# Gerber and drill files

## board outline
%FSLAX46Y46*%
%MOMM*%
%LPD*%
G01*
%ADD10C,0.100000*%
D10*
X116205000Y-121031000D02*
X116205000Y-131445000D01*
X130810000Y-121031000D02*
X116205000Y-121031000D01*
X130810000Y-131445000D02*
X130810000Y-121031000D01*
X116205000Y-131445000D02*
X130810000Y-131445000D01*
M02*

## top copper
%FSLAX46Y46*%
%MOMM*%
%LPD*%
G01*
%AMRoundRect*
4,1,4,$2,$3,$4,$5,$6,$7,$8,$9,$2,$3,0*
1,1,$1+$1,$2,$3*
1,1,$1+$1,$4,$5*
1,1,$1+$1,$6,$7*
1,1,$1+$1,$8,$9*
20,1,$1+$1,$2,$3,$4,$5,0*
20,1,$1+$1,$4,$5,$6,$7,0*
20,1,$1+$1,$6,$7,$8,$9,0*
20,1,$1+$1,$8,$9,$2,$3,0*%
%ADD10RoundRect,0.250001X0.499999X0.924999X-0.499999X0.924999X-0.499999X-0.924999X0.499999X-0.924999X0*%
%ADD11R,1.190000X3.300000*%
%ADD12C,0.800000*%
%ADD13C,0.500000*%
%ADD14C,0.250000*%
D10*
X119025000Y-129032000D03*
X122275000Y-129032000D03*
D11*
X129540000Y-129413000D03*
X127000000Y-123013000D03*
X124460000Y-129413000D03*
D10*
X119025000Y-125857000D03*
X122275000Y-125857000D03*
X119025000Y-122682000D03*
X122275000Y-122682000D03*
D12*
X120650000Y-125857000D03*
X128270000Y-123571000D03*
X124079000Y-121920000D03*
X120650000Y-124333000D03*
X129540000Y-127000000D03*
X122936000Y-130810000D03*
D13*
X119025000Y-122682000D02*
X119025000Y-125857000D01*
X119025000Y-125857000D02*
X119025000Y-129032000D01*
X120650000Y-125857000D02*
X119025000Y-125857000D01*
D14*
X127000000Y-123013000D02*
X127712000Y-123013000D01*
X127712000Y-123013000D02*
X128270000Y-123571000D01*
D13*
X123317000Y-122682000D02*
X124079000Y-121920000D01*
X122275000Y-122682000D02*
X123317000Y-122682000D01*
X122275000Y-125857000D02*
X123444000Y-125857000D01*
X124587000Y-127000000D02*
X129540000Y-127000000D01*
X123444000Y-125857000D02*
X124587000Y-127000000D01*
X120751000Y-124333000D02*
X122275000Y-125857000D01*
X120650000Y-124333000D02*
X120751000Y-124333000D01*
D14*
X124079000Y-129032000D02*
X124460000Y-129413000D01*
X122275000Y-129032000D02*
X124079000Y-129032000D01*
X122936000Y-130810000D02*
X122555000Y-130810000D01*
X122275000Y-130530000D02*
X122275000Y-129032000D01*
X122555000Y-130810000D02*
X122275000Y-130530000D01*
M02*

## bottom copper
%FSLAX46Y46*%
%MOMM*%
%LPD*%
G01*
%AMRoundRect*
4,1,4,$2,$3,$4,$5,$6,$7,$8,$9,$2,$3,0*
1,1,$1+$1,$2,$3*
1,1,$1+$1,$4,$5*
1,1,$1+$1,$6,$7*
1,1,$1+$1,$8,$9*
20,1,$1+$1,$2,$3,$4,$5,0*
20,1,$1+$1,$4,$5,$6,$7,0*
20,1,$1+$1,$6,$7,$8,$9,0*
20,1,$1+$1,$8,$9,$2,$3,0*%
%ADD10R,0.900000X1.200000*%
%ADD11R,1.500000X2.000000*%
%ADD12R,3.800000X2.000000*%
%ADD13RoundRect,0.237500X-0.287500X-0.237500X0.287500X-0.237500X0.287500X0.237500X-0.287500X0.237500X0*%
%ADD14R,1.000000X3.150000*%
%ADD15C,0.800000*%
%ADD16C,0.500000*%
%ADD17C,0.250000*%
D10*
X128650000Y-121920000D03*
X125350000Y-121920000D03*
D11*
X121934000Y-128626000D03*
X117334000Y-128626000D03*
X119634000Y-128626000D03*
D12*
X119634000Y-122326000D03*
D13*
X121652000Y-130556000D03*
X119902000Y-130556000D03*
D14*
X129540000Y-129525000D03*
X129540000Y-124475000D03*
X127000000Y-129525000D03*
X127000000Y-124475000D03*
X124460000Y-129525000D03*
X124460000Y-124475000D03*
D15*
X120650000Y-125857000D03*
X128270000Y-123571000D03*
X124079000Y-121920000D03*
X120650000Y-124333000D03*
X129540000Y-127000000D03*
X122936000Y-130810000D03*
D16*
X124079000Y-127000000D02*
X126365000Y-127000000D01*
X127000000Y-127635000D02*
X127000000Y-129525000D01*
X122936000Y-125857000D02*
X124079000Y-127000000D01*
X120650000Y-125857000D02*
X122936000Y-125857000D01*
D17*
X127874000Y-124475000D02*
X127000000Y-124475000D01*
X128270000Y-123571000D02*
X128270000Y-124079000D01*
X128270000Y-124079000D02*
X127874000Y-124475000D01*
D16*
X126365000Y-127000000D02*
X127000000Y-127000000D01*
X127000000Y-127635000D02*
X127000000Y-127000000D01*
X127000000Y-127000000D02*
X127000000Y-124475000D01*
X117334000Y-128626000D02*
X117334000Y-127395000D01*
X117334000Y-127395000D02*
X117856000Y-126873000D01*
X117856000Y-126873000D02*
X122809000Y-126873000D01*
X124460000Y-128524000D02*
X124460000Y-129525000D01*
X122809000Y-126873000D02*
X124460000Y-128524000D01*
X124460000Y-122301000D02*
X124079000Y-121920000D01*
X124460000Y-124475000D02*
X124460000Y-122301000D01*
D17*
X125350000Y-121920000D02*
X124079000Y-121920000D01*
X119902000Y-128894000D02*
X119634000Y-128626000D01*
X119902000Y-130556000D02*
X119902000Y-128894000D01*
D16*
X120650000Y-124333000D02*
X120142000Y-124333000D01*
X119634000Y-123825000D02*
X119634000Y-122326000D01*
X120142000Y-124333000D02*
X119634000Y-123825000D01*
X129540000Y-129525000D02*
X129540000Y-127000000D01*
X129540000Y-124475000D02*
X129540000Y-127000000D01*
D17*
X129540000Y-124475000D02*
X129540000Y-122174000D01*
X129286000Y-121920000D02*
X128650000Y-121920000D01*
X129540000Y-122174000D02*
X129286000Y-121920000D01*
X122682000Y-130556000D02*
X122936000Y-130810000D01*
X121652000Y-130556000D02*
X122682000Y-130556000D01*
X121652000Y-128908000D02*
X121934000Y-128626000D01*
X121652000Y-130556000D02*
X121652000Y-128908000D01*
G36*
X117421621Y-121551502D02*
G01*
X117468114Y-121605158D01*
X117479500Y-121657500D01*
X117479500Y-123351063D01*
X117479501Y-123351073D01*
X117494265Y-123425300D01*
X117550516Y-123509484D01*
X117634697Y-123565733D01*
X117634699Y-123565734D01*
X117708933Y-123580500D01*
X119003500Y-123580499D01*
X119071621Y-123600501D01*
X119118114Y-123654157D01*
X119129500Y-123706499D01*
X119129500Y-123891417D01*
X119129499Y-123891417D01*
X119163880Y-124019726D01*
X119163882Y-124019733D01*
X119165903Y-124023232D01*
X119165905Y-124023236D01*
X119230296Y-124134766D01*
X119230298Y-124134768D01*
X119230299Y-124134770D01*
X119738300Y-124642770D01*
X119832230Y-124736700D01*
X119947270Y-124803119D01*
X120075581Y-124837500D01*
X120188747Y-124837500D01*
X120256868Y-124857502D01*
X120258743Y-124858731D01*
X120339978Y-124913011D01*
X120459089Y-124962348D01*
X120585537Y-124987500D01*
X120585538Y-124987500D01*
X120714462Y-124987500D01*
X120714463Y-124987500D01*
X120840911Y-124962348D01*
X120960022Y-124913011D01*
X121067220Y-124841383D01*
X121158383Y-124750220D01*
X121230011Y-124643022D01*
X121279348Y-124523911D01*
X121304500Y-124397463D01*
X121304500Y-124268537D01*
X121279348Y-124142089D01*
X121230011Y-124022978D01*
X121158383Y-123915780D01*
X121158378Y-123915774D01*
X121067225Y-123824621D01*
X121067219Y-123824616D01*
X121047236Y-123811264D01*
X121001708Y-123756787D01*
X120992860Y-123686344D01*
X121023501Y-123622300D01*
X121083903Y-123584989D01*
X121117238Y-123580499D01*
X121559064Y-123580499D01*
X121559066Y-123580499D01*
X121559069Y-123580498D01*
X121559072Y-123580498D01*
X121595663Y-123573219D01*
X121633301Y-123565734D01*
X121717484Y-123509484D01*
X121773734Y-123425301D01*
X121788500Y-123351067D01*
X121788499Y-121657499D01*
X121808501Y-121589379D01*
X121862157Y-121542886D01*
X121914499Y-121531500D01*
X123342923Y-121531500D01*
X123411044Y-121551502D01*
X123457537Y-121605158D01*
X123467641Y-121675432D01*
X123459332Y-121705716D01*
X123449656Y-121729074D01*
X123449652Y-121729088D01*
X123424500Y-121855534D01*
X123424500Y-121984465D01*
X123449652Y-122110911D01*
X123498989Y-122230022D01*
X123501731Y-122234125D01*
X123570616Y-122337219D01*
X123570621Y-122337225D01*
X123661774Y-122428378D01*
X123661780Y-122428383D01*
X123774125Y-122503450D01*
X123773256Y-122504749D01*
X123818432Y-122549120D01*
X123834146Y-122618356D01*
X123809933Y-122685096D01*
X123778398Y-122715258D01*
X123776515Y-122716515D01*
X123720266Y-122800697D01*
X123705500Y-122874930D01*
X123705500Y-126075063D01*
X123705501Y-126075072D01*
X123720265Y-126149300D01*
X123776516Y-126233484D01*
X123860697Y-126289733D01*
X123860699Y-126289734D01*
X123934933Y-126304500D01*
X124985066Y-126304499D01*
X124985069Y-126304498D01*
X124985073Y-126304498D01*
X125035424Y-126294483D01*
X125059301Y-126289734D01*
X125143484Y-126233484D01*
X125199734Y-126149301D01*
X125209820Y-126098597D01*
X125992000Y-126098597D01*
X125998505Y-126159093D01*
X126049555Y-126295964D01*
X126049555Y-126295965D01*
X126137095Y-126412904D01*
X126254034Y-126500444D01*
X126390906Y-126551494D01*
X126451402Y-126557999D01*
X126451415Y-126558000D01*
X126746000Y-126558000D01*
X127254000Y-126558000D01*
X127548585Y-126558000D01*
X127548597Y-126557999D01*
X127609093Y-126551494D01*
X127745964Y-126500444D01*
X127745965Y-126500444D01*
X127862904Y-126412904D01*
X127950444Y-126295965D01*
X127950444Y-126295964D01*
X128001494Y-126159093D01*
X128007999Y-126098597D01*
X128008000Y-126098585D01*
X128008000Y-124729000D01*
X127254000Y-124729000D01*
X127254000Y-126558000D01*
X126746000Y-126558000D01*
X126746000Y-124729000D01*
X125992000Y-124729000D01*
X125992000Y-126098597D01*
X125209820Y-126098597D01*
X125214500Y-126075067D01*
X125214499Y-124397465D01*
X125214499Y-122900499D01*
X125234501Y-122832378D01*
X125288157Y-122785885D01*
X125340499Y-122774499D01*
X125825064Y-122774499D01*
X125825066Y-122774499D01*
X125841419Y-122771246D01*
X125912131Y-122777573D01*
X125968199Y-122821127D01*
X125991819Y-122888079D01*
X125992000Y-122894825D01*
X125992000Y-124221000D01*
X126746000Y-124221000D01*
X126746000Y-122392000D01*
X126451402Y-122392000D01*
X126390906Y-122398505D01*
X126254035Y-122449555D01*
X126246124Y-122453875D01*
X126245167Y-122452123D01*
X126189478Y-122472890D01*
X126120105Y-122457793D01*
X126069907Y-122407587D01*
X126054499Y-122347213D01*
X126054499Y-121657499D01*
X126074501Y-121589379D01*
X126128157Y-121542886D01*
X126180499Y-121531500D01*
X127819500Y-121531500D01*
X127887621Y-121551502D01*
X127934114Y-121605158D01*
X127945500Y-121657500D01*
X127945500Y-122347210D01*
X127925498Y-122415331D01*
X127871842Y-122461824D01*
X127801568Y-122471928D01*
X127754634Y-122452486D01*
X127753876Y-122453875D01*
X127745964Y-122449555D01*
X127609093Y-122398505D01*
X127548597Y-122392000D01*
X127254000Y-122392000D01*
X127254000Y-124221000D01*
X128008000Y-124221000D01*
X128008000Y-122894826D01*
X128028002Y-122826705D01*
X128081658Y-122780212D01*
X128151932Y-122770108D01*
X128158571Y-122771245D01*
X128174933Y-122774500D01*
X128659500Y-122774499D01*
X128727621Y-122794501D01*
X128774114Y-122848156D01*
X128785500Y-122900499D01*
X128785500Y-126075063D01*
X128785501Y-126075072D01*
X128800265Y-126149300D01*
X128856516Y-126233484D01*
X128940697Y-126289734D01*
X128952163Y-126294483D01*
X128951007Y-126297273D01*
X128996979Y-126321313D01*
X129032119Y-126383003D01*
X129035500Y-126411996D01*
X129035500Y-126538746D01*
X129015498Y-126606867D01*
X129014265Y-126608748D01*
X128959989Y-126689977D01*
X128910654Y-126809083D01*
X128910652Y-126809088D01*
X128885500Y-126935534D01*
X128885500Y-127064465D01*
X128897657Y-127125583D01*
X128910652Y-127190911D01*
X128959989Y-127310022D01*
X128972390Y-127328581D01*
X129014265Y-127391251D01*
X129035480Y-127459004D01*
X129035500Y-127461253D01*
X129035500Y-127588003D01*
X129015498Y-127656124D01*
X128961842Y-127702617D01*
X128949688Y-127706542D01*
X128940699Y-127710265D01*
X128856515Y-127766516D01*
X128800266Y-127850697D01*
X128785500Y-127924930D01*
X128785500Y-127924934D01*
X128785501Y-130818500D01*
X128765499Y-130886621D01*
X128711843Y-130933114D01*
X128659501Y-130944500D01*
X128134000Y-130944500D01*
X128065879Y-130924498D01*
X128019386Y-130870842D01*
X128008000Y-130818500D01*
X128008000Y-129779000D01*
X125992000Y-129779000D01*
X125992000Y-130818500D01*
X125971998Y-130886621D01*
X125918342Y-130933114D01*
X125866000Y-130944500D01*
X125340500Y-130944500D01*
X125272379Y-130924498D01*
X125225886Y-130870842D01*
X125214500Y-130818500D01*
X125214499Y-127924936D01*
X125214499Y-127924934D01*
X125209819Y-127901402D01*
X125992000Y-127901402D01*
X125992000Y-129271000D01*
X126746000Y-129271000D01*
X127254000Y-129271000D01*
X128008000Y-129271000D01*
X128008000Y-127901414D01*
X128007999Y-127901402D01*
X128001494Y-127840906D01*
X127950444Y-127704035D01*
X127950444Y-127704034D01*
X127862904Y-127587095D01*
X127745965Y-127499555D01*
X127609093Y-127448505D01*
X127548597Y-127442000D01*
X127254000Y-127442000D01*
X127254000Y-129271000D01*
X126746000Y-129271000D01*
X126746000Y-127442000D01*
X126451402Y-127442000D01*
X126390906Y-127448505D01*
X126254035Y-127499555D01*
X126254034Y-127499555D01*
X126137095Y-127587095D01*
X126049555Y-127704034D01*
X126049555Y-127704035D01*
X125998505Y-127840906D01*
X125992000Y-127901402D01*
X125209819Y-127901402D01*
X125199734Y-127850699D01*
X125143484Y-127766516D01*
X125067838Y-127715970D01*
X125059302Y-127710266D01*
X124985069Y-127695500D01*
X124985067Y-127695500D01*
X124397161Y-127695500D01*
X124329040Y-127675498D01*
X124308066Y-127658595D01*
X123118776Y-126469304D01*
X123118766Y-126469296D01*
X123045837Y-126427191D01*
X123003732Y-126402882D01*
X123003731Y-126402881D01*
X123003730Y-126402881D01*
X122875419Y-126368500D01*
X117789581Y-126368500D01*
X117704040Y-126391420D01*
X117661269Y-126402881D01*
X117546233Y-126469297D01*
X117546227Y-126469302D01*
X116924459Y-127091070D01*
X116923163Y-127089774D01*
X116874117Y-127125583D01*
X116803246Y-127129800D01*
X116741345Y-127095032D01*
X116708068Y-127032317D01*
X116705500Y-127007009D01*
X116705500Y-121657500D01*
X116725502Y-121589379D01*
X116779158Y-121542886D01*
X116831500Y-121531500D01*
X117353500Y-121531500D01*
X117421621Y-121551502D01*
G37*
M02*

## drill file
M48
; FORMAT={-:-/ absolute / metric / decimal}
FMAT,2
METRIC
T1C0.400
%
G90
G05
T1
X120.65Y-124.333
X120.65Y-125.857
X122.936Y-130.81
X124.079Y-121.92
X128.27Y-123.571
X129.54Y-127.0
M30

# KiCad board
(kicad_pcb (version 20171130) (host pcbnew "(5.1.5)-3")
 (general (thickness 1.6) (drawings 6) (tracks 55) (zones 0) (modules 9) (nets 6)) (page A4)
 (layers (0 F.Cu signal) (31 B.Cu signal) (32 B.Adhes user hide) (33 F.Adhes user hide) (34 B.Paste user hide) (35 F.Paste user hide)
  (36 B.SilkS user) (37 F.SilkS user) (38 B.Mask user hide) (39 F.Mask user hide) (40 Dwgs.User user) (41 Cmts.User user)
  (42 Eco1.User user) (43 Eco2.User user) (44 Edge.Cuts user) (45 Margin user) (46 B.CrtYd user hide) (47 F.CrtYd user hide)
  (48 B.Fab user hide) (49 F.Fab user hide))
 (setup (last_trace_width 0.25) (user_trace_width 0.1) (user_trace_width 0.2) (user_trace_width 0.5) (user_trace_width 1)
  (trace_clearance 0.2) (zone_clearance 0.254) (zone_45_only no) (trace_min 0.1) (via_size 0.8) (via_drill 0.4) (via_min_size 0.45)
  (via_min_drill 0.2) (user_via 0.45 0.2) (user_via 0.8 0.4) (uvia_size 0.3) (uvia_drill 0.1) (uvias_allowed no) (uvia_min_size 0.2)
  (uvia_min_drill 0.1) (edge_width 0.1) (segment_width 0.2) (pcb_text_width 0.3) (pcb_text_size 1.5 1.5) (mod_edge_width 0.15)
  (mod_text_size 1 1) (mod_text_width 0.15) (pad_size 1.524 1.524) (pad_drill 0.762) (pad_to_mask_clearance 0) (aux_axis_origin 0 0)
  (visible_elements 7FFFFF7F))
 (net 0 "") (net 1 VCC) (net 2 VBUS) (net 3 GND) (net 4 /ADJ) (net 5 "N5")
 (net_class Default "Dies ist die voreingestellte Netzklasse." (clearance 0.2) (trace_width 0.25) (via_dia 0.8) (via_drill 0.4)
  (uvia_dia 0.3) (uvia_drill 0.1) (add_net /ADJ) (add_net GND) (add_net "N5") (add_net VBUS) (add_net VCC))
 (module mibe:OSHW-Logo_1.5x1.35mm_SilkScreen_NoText (layer F.Cu) (at 117.348 130.429)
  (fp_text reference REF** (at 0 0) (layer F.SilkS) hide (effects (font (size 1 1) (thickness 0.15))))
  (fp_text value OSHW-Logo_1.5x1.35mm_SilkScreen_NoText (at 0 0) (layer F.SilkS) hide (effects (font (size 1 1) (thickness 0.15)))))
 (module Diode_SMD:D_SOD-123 (layer B.Cu) (at 127 121.92)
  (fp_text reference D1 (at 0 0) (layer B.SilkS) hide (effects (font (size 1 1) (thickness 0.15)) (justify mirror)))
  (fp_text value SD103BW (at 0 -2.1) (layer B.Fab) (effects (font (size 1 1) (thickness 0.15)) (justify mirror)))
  (pad 2 smd rect (at 1.65 0) (size 0.9 1.2) (layers B.Cu B.Paste B.Mask) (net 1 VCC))
  (pad 1 smd rect (at -1.65 0) (size 0.9 1.2) (layers B.Cu B.Paste B.Mask) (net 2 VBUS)))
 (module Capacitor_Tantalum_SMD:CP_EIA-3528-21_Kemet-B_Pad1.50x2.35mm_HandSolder (layer F.Cu) (at 120.65 129.032 180)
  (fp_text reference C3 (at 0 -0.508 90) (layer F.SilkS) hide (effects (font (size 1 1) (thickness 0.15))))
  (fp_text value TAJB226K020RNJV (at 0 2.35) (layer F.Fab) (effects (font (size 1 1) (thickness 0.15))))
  (pad 2 smd roundrect (at 1.625 0 180) (size 1.5 2.35) (layers F.Cu F.Paste F.Mask) (roundrect_rratio 0.166667) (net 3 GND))
  (pad 1 smd roundrect (at -1.625 0 180) (size 1.5 2.35) (layers F.Cu F.Paste F.Mask) (roundrect_rratio 0.166667) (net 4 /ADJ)))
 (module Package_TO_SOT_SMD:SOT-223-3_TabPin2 (layer B.Cu) (at 119.634 125.476 90)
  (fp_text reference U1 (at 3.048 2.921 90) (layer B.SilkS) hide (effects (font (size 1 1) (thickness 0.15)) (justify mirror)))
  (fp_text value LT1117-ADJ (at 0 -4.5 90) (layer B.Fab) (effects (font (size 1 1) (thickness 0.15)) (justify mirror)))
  (pad 1 smd rect (at -3.15 2.3 90) (size 2 1.5) (layers B.Cu B.Paste B.Mask) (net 4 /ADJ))
  (pad 3 smd rect (at -3.15 -2.3 90) (size 2 1.5) (layers B.Cu B.Paste B.Mask) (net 2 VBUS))
  (pad 2 smd rect (at -3.15 0 90) (size 2 1.5) (layers B.Cu B.Paste B.Mask) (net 1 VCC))
  (pad 2 smd rect (at 3.15 0 90) (size 2 3.8) (layers B.Cu B.Paste B.Mask) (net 1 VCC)))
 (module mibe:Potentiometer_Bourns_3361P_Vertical (layer F.Cu) (at 127 126.213 180)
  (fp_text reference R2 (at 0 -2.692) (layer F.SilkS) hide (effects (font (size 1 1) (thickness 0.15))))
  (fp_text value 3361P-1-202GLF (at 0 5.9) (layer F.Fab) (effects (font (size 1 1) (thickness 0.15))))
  (pad 3 smd rect (at -2.54 -3.2 180) (size 1.19 3.3) (layers F.Cu F.Paste F.Mask) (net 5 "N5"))
  (pad 2 smd rect (at 0 3.2 180) (size 1.19 3.3) (layers F.Cu F.Paste F.Mask) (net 3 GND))
  (pad 1 smd rect (at 2.54 -3.2 180) (size 1.19 3.3) (layers F.Cu F.Paste F.Mask) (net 4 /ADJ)))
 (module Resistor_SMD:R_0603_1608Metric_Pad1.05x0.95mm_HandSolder (layer B.Cu) (at 120.777 130.556)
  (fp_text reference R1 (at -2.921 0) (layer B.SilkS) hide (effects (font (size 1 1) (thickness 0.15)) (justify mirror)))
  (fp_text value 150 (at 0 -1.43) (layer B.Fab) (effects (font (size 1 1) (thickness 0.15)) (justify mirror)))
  (pad 2 smd roundrect (at 0.875 0) (size 1.05 0.95) (layers B.Cu B.Paste B.Mask) (roundrect_rratio 0.25) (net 4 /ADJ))
  (pad 1 smd roundrect (at -0.875 0) (size 1.05 0.95) (layers B.Cu B.Paste B.Mask) (roundrect_rratio 0.25) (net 1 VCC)))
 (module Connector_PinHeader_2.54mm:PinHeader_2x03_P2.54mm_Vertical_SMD (layer B.Cu) (at 127 127 270)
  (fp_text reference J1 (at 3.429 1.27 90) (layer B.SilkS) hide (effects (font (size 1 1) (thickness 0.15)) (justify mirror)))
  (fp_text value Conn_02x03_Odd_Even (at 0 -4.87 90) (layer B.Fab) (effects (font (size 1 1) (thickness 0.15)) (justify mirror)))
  (pad 6 smd rect (at 2.525 -2.54 270) (size 3.15 1) (layers B.Cu B.Paste B.Mask) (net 1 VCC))
  (pad 5 smd rect (at -2.525 -2.54 270) (size 3.15 1) (layers B.Cu B.Paste B.Mask) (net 1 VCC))
  (pad 4 smd rect (at 2.525 0 270) (size 3.15 1) (layers B.Cu B.Paste B.Mask) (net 3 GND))
  (pad 3 smd rect (at -2.525 0 270) (size 3.15 1) (layers B.Cu B.Paste B.Mask) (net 3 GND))
  (pad 2 smd rect (at 2.525 2.54 270) (size 3.15 1) (layers B.Cu B.Paste B.Mask) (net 2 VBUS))
  (pad 1 smd rect (at -2.525 2.54 270) (size 3.15 1) (layers B.Cu B.Paste B.Mask) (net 2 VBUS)))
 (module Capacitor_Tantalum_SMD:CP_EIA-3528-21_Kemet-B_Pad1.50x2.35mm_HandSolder (layer F.Cu) (at 120.65 125.857 180)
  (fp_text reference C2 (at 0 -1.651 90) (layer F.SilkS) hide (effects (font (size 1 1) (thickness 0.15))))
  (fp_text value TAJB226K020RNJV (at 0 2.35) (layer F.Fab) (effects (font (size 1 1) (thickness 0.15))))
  (pad 2 smd roundrect (at 1.625 0 180) (size 1.5 2.35) (layers F.Cu F.Paste F.Mask) (roundrect_rratio 0.166667) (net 3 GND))
  (pad 1 smd roundrect (at -1.625 0 180) (size 1.5 2.35) (layers F.Cu F.Paste F.Mask) (roundrect_rratio 0.166667) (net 1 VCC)))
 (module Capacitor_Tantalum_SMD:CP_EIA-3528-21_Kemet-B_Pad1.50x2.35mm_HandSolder (layer F.Cu) (at 120.65 122.682 180)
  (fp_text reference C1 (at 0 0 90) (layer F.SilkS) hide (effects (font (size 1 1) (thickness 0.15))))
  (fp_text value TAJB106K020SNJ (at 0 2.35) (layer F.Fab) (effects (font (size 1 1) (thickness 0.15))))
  (pad 2 smd roundrect (at 1.625 0 180) (size 1.5 2.35) (layers F.Cu F.Paste F.Mask) (roundrect_rratio 0.166667) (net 3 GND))
  (pad 1 smd roundrect (at -1.625 0 180) (size 1.5 2.35) (layers F.Cu F.Paste F.Mask) (roundrect_rratio 0.166667) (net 2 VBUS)))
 (gr_line (start 116.205 121.031) (end 116.205 131.445) (layer Edge.Cuts) (width 0.1))
 (gr_line (start 130.81 121.031) (end 116.205 121.031) (layer Edge.Cuts) (width 0.1))
 (gr_line (start 130.81 131.445) (end 130.81 121.031) (layer Edge.Cuts) (width 0.1))
 (gr_line (start 116.205 131.445) (end 130.81 131.445) (layer Edge.Cuts) (width 0.1))
 (segment (start 119.025 122.682) (end 119.025 125.857) (width 0.5) (layer F.Cu) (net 3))
 (segment (start 119.025 125.857) (end 119.025 129.032) (width 0.5) (layer F.Cu) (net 3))
 (segment (start 124.079 127) (end 126.365 127) (width 0.5) (layer B.Cu) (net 3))
 (segment (start 127 127.635) (end 127 129.525) (width 0.5) (layer B.Cu) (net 3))
 (via (at 120.65 125.857) (size 0.8) (drill 0.4) (layers F.Cu B.Cu) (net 3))
 (segment (start 120.65 125.857) (end 119.025 125.857) (width 0.5) (layer F.Cu) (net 3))
 (segment (start 122.936 125.857) (end 124.079 127) (width 0.5) (layer B.Cu) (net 3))
 (segment (start 120.65 125.857) (end 122.936 125.857) (width 0.5) (layer B.Cu) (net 3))
 (via (at 128.27 123.571) (size 0.8) (drill 0.4) (layers F.Cu B.Cu) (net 3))
 (segment (start 127 123.013) (end 127.712 123.013) (width 0.25) (layer F.Cu) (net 3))
 (segment (start 127.712 123.013) (end 128.27 123.571) (width 0.25) (layer F.Cu) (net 3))
 (segment (start 127.874 124.475) (end 127 124.475) (width 0.25) (layer B.Cu) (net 3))
 (segment (start 128.27 123.571) (end 128.27 124.079) (width 0.25) (layer B.Cu) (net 3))
 (segment (start 128.27 124.079) (end 127.874 124.475) (width 0.25) (layer B.Cu) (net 3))
 (segment (start 126.365 127) (end 127 127) (width 0.5) (layer B.Cu) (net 3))
 (segment (start 127 127.635) (end 127 127) (width 0.5) (layer B.Cu) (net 3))
 (segment (start 127 127) (end 127 124.475) (width 0.5) (layer B.Cu) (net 3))
 (via (at 124.079 121.92) (size 0.8) (drill 0.4) (layers F.Cu B.Cu) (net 2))
 (segment (start 117.334 128.626) (end 117.334 127.395) (width 0.5) (layer B.Cu) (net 2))
 (segment (start 117.334 127.395) (end 117.856 126.873) (width 0.5) (layer B.Cu) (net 2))
 (segment (start 117.856 126.873) (end 122.809 126.873) (width 0.5) (layer B.Cu) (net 2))
 (segment (start 124.46 128.524) (end 124.46 129.525) (width 0.5) (layer B.Cu) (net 2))
 (segment (start 122.809 126.873) (end 124.46 128.524) (width 0.5) (layer B.Cu) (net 2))
 (segment (start 124.46 122.301) (end 124.079 121.92) (width 0.5) (layer B.Cu) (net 2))
 (segment (start 124.46 124.475) (end 124.46 122.301) (width 0.5) (layer B.Cu) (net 2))
 (segment (start 125.35 121.92) (end 124.079 121.92) (width 0.25) (layer B.Cu) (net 2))
 (segment (start 123.317 122.682) (end 124.079 121.92) (width 0.5) (layer F.Cu) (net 2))
 (segment (start 122.275 122.682) (end 123.317 122.682) (width 0.5) (layer F.Cu) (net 2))
 (via (at 120.65 124.333) (size 0.8) (drill 0.4) (layers F.Cu B.Cu) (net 1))
 (via (at 129.54 127) (size 0.8) (drill 0.4) (layers F.Cu B.Cu) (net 1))
 (segment (start 119.902 128.894) (end 119.634 128.626) (width 0.25) (layer B.Cu) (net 1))
 (segment (start 119.902 130.556) (end 119.902 128.894) (width 0.25) (layer B.Cu) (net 1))
 (segment (start 122.275 125.857) (end 123.444 125.857) (width 0.5) (layer F.Cu) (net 1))
 (segment (start 124.587 127) (end 129.54 127) (width 0.5) (layer F.Cu) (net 1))
 (segment (start 123.444 125.857) (end 124.587 127) (width 0.5) (layer F.Cu) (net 1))
 (segment (start 120.65 124.333) (end 120.142 124.333) (width 0.5) (layer B.Cu) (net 1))
 (segment (start 119.634 123.825) (end 119.634 122.326) (width 0.5) (layer B.Cu) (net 1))
 (segment (start 120.142 124.333) (end 119.634 123.825) (width 0.5) (layer B.Cu) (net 1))
 (segment (start 129.54 129.525) (end 129.54 127) (width 0.5) (layer B.Cu) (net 1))
 (segment (start 129.54 124.475) (end 129.54 127) (width 0.5) (layer B.Cu) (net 1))
 (segment (start 129.54 124.475) (end 129.54 122.174) (width 0.25) (layer B.Cu) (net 1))
 (segment (start 129.286 121.92) (end 128.65 121.92) (width 0.25) (layer B.Cu) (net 1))
 (segment (start 129.54 122.174) (end 129.286 121.92) (width 0.25) (layer B.Cu) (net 1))
 (segment (start 120.751 124.333) (end 122.275 125.857) (width 0.5) (layer F.Cu) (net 1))
 (segment (start 120.65 124.333) (end 120.751 124.333) (width 0.5) (layer F.Cu) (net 1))
 (via (at 122.936 130.81) (size 0.8) (drill 0.4) (layers F.Cu B.Cu) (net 4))
 (segment (start 124.079 129.032) (end 124.46 129.413) (width 0.25) (layer F.Cu) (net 4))
 (segment (start 122.275 129.032) (end 124.079 129.032) (width 0.25) (layer F.Cu) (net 4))
 (segment (start 122.936 130.81) (end 122.555 130.81) (width 0.25) (layer F.Cu) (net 4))
 (segment (start 122.275 130.53) (end 122.275 129.032) (width 0.25) (layer F.Cu) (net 4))
 (segment (start 122.555 130.81) (end 122.275 130.53) (width 0.25) (layer F.Cu) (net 4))
 (segment (start 122.682 130.556) (end 122.936 130.81) (width 0.25) (layer B.Cu) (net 4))
 (segment (start 121.652 130.556) (end 122.682 130.556) (width 0.25) (layer B.Cu) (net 4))
 (segment (start 121.652 128.908) (end 121.934 128.626) (width 0.25) (layer B.Cu) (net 4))
 (segment (start 121.652 130.556) (end 121.652 128.908) (width 0.25) (layer B.Cu) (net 4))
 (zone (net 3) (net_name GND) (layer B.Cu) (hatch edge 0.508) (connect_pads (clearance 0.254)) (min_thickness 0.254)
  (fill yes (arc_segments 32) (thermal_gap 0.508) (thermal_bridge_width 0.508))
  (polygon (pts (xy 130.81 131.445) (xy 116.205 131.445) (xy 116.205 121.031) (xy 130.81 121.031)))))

